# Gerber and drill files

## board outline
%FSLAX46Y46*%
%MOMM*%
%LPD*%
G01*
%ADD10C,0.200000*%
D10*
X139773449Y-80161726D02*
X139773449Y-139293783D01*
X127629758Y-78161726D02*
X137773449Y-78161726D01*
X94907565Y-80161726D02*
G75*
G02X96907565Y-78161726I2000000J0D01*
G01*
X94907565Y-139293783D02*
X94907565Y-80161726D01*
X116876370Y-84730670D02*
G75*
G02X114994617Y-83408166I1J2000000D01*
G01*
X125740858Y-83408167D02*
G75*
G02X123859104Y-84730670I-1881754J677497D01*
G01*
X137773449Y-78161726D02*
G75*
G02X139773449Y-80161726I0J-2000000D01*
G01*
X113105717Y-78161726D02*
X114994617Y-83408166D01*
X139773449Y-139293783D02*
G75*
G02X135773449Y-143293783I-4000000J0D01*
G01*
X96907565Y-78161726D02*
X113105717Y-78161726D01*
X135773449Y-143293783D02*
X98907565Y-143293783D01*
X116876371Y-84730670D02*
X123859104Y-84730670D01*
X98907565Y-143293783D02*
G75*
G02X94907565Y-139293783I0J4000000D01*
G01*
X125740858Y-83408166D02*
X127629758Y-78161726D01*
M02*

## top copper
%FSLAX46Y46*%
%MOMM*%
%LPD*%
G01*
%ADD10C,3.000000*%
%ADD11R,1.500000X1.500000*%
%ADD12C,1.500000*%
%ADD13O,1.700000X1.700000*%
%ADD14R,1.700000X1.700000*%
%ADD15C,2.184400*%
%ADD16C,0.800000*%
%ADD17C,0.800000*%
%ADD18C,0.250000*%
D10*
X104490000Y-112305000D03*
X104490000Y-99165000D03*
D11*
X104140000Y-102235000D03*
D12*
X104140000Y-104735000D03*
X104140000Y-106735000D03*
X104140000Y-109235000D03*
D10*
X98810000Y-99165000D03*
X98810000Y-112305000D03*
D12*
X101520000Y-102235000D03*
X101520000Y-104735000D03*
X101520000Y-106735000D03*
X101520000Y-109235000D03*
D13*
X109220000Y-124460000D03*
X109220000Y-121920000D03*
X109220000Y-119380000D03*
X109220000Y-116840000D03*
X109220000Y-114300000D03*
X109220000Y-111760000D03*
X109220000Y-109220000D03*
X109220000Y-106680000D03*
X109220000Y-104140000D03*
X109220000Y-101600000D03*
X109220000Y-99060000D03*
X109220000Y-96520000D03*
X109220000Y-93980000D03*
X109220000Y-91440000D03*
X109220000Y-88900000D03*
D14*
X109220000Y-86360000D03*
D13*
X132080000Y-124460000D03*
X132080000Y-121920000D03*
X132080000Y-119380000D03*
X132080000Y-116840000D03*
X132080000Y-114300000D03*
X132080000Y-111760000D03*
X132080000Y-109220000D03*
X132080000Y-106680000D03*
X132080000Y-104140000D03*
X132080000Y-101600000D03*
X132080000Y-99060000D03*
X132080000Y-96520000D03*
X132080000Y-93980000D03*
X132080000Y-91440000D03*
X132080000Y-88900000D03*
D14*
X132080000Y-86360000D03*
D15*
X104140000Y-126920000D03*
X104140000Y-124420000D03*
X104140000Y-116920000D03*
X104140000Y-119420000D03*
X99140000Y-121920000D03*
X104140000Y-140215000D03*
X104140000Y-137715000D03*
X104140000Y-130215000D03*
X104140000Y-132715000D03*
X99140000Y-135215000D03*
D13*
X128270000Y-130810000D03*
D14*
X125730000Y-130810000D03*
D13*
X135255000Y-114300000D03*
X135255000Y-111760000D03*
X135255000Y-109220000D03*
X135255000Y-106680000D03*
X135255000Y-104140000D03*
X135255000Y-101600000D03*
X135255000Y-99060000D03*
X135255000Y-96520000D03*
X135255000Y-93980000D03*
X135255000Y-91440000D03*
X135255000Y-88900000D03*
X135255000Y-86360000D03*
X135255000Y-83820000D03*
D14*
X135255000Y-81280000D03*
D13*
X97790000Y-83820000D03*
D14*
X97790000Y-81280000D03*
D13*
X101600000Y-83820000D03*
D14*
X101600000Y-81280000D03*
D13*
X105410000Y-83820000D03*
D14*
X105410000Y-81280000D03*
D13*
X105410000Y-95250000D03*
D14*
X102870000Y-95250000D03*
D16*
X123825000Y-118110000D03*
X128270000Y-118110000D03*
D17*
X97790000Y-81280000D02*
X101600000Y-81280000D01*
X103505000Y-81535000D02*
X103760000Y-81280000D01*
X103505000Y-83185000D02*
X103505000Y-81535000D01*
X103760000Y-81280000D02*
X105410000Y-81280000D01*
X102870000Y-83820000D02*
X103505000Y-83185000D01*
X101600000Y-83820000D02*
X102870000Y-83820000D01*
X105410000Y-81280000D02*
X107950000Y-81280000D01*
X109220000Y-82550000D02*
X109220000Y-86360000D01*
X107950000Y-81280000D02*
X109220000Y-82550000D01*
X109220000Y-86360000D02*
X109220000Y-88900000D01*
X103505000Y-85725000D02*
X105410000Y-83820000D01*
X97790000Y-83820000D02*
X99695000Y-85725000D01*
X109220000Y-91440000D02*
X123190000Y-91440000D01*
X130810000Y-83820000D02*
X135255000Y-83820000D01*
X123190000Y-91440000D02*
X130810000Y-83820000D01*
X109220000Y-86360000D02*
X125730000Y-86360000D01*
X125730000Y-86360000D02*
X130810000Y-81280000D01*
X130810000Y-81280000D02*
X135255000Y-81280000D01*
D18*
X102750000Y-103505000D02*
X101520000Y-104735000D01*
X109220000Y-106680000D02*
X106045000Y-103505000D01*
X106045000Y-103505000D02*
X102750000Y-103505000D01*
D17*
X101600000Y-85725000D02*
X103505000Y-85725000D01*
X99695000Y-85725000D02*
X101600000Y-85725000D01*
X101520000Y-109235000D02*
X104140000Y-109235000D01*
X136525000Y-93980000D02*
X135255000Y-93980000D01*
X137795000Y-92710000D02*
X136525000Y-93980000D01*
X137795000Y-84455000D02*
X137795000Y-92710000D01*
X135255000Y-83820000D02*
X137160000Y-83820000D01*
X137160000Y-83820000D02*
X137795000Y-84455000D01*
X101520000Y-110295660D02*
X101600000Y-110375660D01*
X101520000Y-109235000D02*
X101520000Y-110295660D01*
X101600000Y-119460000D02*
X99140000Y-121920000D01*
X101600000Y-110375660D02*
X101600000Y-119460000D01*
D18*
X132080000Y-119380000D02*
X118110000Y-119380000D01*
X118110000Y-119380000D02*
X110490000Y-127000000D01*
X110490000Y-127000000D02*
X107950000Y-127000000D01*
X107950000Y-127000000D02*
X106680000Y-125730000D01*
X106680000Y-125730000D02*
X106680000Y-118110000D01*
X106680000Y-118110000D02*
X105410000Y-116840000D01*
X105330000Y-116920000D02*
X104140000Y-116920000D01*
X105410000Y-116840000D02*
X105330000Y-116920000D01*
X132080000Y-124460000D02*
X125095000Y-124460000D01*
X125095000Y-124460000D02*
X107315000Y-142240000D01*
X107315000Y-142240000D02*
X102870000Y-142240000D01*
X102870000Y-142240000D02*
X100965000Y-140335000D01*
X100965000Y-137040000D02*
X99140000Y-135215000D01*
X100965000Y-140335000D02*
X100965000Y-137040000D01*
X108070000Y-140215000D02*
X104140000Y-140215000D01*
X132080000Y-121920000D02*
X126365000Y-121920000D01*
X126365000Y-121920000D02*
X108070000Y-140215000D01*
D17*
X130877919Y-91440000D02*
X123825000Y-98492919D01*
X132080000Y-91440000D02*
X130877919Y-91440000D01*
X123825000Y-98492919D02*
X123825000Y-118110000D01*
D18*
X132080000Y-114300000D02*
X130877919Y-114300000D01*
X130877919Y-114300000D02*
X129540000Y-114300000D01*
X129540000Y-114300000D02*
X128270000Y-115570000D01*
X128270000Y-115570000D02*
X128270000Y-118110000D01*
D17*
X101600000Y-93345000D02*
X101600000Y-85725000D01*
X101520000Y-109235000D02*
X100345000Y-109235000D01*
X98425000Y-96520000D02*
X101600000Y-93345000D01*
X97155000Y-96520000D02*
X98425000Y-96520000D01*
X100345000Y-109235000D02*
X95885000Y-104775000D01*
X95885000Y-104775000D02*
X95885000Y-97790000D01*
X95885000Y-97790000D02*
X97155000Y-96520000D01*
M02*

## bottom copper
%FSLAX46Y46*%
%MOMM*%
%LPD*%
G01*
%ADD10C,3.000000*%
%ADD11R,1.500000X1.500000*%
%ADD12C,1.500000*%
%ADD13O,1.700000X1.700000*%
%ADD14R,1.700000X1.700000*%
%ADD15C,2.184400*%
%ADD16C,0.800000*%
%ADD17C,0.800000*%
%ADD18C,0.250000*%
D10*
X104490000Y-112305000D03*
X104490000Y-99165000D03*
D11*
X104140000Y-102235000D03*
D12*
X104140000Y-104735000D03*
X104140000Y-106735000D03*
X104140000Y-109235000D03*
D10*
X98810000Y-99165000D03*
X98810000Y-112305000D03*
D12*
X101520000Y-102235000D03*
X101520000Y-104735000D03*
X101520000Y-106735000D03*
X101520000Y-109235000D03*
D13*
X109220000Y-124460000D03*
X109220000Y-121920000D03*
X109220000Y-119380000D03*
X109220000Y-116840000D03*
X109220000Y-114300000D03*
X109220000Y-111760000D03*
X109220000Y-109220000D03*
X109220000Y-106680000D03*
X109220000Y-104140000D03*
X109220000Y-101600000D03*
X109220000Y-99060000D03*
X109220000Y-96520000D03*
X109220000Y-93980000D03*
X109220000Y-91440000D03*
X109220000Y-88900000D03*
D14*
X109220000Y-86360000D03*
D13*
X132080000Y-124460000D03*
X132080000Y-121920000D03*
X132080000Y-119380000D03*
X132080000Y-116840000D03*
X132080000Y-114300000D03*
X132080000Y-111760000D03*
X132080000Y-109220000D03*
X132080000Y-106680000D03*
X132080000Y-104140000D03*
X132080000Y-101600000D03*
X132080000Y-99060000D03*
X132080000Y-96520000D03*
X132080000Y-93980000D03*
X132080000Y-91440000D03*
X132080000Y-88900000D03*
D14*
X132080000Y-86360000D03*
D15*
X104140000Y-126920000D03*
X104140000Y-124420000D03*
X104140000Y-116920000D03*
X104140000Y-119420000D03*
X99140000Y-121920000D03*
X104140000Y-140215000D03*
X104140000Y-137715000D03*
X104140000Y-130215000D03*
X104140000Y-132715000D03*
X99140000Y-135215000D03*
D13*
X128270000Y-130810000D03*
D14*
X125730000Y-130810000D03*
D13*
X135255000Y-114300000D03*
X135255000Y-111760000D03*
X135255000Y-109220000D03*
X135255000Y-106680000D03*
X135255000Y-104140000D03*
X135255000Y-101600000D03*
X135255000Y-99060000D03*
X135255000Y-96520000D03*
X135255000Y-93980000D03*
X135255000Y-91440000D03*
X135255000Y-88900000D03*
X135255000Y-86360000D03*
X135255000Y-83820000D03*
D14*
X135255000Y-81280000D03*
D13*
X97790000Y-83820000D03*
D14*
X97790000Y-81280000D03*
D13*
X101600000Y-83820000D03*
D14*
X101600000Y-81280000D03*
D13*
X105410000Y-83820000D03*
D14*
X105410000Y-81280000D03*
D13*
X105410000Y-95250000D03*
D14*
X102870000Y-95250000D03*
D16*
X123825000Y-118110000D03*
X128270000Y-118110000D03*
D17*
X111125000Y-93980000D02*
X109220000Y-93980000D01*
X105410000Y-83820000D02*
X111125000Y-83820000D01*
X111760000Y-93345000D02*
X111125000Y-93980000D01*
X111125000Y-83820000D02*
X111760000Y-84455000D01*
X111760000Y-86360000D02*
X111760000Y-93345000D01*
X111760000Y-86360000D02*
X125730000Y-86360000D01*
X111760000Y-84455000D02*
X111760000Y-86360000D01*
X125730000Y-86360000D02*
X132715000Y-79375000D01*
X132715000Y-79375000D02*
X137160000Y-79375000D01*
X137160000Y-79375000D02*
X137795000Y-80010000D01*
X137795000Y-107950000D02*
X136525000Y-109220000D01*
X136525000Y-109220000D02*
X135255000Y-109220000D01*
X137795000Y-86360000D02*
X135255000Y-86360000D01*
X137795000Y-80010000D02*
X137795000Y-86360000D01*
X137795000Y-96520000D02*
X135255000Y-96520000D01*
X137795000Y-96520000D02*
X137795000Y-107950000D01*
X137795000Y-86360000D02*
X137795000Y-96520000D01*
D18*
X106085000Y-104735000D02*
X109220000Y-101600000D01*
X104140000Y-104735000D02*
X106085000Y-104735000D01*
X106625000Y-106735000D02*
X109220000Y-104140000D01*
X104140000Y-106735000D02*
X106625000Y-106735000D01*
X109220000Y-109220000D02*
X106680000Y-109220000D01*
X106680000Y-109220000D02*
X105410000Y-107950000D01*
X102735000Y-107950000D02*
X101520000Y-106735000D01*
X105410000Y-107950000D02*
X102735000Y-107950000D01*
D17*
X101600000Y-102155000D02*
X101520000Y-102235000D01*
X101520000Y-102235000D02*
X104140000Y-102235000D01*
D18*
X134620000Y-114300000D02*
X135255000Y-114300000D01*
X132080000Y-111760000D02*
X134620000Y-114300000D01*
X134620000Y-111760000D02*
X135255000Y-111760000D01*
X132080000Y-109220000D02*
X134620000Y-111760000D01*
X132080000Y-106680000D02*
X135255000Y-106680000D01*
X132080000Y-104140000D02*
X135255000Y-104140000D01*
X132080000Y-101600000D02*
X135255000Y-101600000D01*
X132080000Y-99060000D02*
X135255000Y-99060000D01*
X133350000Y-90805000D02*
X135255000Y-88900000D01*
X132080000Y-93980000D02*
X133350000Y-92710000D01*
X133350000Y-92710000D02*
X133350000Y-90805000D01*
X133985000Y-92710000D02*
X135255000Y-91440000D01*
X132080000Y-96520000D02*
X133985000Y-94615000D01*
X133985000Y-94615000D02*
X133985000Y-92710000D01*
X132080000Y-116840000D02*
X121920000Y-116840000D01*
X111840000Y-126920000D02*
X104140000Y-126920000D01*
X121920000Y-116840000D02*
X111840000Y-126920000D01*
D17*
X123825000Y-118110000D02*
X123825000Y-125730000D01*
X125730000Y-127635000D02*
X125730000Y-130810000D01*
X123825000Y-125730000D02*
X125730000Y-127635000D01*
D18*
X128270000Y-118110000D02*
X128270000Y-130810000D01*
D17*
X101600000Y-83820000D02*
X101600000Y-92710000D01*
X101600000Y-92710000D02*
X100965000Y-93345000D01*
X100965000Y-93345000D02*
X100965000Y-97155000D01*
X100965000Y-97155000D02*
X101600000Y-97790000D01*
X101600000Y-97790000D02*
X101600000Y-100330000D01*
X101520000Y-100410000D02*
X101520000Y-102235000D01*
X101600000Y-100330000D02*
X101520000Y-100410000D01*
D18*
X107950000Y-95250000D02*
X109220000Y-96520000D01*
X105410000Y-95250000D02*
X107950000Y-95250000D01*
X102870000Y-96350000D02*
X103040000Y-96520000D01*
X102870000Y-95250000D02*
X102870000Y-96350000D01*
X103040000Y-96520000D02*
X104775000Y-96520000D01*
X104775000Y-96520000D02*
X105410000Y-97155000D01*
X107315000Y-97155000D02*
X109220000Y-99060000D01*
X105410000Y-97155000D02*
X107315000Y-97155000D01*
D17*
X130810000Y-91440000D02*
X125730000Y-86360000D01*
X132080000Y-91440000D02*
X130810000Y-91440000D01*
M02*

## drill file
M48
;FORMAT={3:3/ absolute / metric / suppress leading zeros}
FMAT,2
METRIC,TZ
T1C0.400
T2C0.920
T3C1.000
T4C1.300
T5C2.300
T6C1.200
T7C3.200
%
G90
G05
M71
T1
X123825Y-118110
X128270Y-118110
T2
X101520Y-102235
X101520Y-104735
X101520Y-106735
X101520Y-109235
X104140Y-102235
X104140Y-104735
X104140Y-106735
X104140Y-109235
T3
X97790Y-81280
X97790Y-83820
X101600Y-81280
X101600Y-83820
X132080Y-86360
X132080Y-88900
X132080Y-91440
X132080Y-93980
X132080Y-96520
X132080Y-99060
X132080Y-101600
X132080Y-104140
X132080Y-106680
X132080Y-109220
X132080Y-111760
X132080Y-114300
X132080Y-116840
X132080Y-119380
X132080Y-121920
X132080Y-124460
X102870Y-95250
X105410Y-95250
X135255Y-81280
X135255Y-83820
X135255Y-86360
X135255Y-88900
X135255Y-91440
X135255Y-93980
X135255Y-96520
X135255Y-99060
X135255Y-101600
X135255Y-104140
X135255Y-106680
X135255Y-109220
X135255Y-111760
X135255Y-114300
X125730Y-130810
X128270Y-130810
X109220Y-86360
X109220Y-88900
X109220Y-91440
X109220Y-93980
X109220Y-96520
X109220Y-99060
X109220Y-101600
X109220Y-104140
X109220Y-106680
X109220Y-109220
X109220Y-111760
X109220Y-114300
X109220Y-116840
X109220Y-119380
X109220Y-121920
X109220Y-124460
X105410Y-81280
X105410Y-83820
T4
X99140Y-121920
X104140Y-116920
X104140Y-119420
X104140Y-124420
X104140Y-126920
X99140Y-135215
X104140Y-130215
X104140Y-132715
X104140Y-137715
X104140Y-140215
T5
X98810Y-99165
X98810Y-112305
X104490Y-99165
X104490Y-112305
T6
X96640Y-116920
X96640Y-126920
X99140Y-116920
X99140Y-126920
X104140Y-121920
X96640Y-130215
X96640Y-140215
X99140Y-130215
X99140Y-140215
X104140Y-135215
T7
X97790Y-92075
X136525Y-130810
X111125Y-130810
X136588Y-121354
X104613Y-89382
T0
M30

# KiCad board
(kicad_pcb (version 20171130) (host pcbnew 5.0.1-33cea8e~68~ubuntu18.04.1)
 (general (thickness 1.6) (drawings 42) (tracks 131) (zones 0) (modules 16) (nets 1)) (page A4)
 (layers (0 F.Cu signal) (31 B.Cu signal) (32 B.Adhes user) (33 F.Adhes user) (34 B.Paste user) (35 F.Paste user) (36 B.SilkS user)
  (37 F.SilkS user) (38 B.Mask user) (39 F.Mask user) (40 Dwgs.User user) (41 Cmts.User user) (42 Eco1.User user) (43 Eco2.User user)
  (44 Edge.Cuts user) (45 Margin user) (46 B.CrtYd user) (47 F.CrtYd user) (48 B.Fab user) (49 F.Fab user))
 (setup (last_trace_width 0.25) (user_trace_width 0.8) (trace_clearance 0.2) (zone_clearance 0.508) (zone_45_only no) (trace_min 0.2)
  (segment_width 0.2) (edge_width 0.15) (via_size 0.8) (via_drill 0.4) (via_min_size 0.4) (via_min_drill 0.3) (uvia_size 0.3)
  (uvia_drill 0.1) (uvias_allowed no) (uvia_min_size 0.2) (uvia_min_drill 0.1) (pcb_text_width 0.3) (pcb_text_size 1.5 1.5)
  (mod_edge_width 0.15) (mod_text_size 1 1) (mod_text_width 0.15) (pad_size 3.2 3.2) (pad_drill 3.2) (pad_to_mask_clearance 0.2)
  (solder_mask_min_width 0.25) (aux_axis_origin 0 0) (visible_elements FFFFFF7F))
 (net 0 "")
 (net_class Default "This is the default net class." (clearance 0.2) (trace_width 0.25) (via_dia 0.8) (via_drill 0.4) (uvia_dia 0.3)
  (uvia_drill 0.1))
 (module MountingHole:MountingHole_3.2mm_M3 (layer F.Cu) (at 97.79 92.075)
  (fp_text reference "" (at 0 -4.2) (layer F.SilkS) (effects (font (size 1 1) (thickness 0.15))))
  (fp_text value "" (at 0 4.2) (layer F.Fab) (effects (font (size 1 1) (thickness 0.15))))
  (pad 1 np_thru_hole circle (at 0 0) (size 3.2 3.2) (drill 3.2) (layers *.Cu *.Mask)))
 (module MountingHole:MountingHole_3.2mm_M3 (layer F.Cu) (at 136.525 130.81)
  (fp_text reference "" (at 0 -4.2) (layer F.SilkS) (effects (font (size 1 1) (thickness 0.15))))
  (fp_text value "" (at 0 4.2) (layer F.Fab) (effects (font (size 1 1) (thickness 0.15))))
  (pad 1 np_thru_hole circle (at 0 0) (size 3.2 3.2) (drill 3.2) (layers *.Cu *.Mask)))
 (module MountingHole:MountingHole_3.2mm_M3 (layer F.Cu) (at 111.125 130.81)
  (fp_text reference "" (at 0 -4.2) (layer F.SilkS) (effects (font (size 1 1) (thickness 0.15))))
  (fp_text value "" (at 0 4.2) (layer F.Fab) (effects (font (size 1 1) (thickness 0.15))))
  (pad 1 np_thru_hole circle (at 0 0) (size 3.2 3.2) (drill 3.2) (layers *.Cu *.Mask)))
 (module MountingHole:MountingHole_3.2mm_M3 (layer F.Cu) (at 136.587912 121.353509)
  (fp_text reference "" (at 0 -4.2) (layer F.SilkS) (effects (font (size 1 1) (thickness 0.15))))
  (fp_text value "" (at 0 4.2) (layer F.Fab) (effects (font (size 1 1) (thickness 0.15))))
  (pad 1 np_thru_hole circle (at 0 0) (size 3.2 3.2) (drill 3.2) (layers *.Cu *.Mask)))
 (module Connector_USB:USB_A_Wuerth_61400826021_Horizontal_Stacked (layer F.Cu) (at 104.14 102.235 270)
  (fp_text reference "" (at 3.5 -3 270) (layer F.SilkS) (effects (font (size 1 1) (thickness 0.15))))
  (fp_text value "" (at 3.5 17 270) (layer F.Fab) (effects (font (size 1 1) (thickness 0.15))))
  (pad 9 thru_hole circle (at 10.07 -0.35 270) (size 3 3) (drill 2.3) (layers *.Cu *.Mask))
  (pad 9 thru_hole circle (at -3.07 -0.35 270) (size 3 3) (drill 2.3) (layers *.Cu *.Mask))
  (pad 1 thru_hole rect (at 0 0 270) (size 1.5 1.5) (drill 0.92) (layers *.Cu *.Mask))
  (pad 2 thru_hole circle (at 2.5 0 270) (size 1.5 1.5) (drill 0.92) (layers *.Cu *.Mask))
  (pad 3 thru_hole circle (at 4.5 0 270) (size 1.5 1.5) (drill 0.92) (layers *.Cu *.Mask))
  (pad 4 thru_hole circle (at 7 0 270) (size 1.5 1.5) (drill 0.92) (layers *.Cu *.Mask))
  (pad 9 thru_hole circle (at -3.07 5.33 270) (size 3 3) (drill 2.3) (layers *.Cu *.Mask))
  (pad 9 thru_hole circle (at 10.07 5.33 270) (size 3 3) (drill 2.3) (layers *.Cu *.Mask))
  (pad 5 thru_hole circle (at 0 2.62 270) (size 1.5 1.5) (drill 0.92) (layers *.Cu *.Mask))
  (pad 6 thru_hole circle (at 2.5 2.62 270) (size 1.5 1.5) (drill 0.92) (layers *.Cu *.Mask))
  (pad 7 thru_hole circle (at 4.5 2.62 270) (size 1.5 1.5) (drill 0.92) (layers *.Cu *.Mask))
  (pad 8 thru_hole circle (at 7 2.62 270) (size 1.5 1.5) (drill 0.92) (layers *.Cu *.Mask)))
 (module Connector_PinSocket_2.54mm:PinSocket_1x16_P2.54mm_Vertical (layer F.Cu) (at 109.22 86.36)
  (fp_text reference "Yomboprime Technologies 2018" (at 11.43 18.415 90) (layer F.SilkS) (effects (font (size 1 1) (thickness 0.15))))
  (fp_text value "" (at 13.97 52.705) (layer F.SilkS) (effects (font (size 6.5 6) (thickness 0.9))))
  (pad 16 thru_hole oval (at 0 38.1) (size 1.7 1.7) (drill 1) (layers *.Cu *.Mask))
  (pad 15 thru_hole oval (at 0 35.56) (size 1.7 1.7) (drill 1) (layers *.Cu *.Mask))
  (pad 14 thru_hole oval (at 0 33.02) (size 1.7 1.7) (drill 1) (layers *.Cu *.Mask))
  (pad 13 thru_hole oval (at 0 30.48) (size 1.7 1.7) (drill 1) (layers *.Cu *.Mask))
  (pad 12 thru_hole oval (at 0 27.94) (size 1.7 1.7) (drill 1) (layers *.Cu *.Mask))
  (pad 11 thru_hole oval (at 0 25.4) (size 1.7 1.7) (drill 1) (layers *.Cu *.Mask))
  (pad 10 thru_hole oval (at 0 22.86) (size 1.7 1.7) (drill 1) (layers *.Cu *.Mask))
  (pad 9 thru_hole oval (at 0 20.32) (size 1.7 1.7) (drill 1) (layers *.Cu *.Mask))
  (pad 8 thru_hole oval (at 0 17.78) (size 1.7 1.7) (drill 1) (layers *.Cu *.Mask))
  (pad 7 thru_hole oval (at 0 15.24) (size 1.7 1.7) (drill 1) (layers *.Cu *.Mask))
  (pad 6 thru_hole oval (at 0 12.7) (size 1.7 1.7) (drill 1) (layers *.Cu *.Mask))
  (pad 5 thru_hole oval (at 0 10.16) (size 1.7 1.7) (drill 1) (layers *.Cu *.Mask))
  (pad 4 thru_hole oval (at 0 7.62) (size 1.7 1.7) (drill 1) (layers *.Cu *.Mask))
  (pad 3 thru_hole oval (at 0 5.08) (size 1.7 1.7) (drill 1) (layers *.Cu *.Mask))
  (pad 2 thru_hole oval (at 0 2.54) (size 1.7 1.7) (drill 1) (layers *.Cu *.Mask))
  (pad 1 thru_hole rect (at 0 0) (size 1.7 1.7) (drill 1) (layers *.Cu *.Mask)))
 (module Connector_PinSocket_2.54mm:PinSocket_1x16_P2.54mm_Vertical (layer F.Cu) (at 132.08 86.36)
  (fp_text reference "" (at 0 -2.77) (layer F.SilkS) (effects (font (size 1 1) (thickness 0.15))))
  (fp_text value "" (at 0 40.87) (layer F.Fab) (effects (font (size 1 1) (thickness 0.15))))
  (pad 16 thru_hole oval (at 0 38.1) (size 1.7 1.7) (drill 1) (layers *.Cu *.Mask))
  (pad 15 thru_hole oval (at 0 35.56) (size 1.7 1.7) (drill 1) (layers *.Cu *.Mask))
  (pad 14 thru_hole oval (at 0 33.02) (size 1.7 1.7) (drill 1) (layers *.Cu *.Mask))
  (pad 13 thru_hole oval (at 0 30.48) (size 1.7 1.7) (drill 1) (layers *.Cu *.Mask))
  (pad 12 thru_hole oval (at 0 27.94) (size 1.7 1.7) (drill 1) (layers *.Cu *.Mask))
  (pad 11 thru_hole oval (at 0 25.4) (size 1.7 1.7) (drill 1) (layers *.Cu *.Mask))
  (pad 10 thru_hole oval (at 0 22.86) (size 1.7 1.7) (drill 1) (layers *.Cu *.Mask))
  (pad 9 thru_hole oval (at 0 20.32) (size 1.7 1.7) (drill 1) (layers *.Cu *.Mask))
  (pad 8 thru_hole oval (at 0 17.78) (size 1.7 1.7) (drill 1) (layers *.Cu *.Mask))
  (pad 7 thru_hole oval (at 0 15.24) (size 1.7 1.7) (drill 1) (layers *.Cu *.Mask))
  (pad 6 thru_hole oval (at 0 12.7) (size 1.7 1.7) (drill 1) (layers *.Cu *.Mask))
  (pad 5 thru_hole oval (at 0 10.16) (size 1.7 1.7) (drill 1) (layers *.Cu *.Mask))
  (pad 4 thru_hole oval (at 0 7.62) (size 1.7 1.7) (drill 1) (layers *.Cu *.Mask))
  (pad 3 thru_hole oval (at 0 5.08) (size 1.7 1.7) (drill 1) (layers *.Cu *.Mask))
  (pad 2 thru_hole oval (at 0 2.54) (size 1.7 1.7) (drill 1) (layers *.Cu *.Mask))
  (pad 1 thru_hole rect (at 0 0) (size 1.7 1.7) (drill 1) (layers *.Cu *.Mask)))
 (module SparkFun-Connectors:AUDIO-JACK (layer F.Cu) (at 99.14 121.92)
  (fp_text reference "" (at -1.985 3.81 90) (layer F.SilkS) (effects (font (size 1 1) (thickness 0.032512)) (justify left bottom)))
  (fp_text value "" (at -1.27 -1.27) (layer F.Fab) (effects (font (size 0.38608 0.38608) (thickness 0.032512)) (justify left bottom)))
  (pad "" np_thru_hole circle (at 5 0) (size 1.2 1.2) (drill 1.2) (layers *.Cu))
  (pad "" np_thru_hole circle (at 0 5) (size 1.2 1.2) (drill 1.2) (layers *.Cu))
  (pad "" np_thru_hole circle (at -2.5 5) (size 1.2 1.2) (drill 1.2) (layers *.Cu))
  (pad "" np_thru_hole circle (at -2.5 -5) (size 1.2 1.2) (drill 1.2) (layers *.Cu))
  (pad "" np_thru_hole circle (at 0 -5) (size 1.2 1.2) (drill 1.2) (layers *.Cu))
  (pad TIP thru_hole circle (at 5 5) (size 2.1844 2.1844) (drill 1.3) (layers *.Cu *.Mask) (solder_mask_margin 0.1016))
  (pad TSH thru_hole circle (at 5 2.5) (size 2.1844 2.1844) (drill 1.3) (layers *.Cu *.Mask) (solder_mask_margin 0.1016))
  (pad RING thru_hole circle (at 5 -5) (size 2.1844 2.1844) (drill 1.3) (layers *.Cu *.Mask) (solder_mask_margin 0.1016))
  (pad RSH thru_hole circle (at 5 -2.5) (size 2.1844 2.1844) (drill 1.3) (layers *.Cu *.Mask) (solder_mask_margin 0.1016))
  (pad SLEEVE thru_hole circle (at 0 0) (size 2.1844 2.1844) (drill 1.3) (layers *.Cu *.Mask) (solder_mask_margin 0.1016)))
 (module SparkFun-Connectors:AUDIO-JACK (layer F.Cu) (at 99.14 135.215)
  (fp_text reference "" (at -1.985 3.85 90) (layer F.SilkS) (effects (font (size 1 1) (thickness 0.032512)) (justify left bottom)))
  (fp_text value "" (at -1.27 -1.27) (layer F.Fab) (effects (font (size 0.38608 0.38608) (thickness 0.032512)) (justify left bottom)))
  (pad "" np_thru_hole circle (at 5 0) (size 1.2 1.2) (drill 1.2) (layers *.Cu))
  (pad "" np_thru_hole circle (at 0 5) (size 1.2 1.2) (drill 1.2) (layers *.Cu))
  (pad "" np_thru_hole circle (at -2.5 5) (size 1.2 1.2) (drill 1.2) (layers *.Cu))
  (pad "" np_thru_hole circle (at -2.5 -5) (size 1.2 1.2) (drill 1.2) (layers *.Cu))
  (pad "" np_thru_hole circle (at 0 -5) (size 1.2 1.2) (drill 1.2) (layers *.Cu))
  (pad TIP thru_hole circle (at 5 5) (size 2.1844 2.1844) (drill 1.3) (layers *.Cu *.Mask) (solder_mask_margin 0.1016))
  (pad TSH thru_hole circle (at 5 2.5) (size 2.1844 2.1844) (drill 1.3) (layers *.Cu *.Mask) (solder_mask_margin 0.1016))
  (pad RING thru_hole circle (at 5 -5) (size 2.1844 2.1844) (drill 1.3) (layers *.Cu *.Mask) (solder_mask_margin 0.1016))
  (pad RSH thru_hole circle (at 5 -2.5) (size 2.1844 2.1844) (drill 1.3) (layers *.Cu *.Mask) (solder_mask_margin 0.1016))
  (pad SLEEVE thru_hole circle (at 0 0) (size 2.1844 2.1844) (drill 1.3) (layers *.Cu *.Mask) (solder_mask_margin 0.1016)))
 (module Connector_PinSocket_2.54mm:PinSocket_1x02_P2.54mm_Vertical (layer F.Cu) (at 125.73 130.81 90)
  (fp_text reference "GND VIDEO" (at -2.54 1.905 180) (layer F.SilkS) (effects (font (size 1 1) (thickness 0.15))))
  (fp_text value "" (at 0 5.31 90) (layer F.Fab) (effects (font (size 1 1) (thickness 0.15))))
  (pad 2 thru_hole oval (at 0 2.54 90) (size 1.7 1.7) (drill 1) (layers *.Cu *.Mask))
  (pad 1 thru_hole rect (at 0 0 90) (size 1.7 1.7) (drill 1) (layers *.Cu *.Mask)))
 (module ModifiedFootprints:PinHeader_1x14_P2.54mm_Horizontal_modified (layer F.Cu) (at 135.255 81.28)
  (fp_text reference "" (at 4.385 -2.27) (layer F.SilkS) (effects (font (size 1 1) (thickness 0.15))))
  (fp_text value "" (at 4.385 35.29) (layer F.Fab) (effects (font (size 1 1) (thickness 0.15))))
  (pad 14 thru_hole oval (at 0 33.02) (size 1.7 1.7) (drill 1) (layers *.Cu *.Mask))
  (pad 13 thru_hole oval (at 0 30.48) (size 1.7 1.7) (drill 1) (layers *.Cu *.Mask))
  (pad 12 thru_hole oval (at 0 27.94) (size 1.7 1.7) (drill 1) (layers *.Cu *.Mask))
  (pad 11 thru_hole oval (at 0 25.4) (size 1.7 1.7) (drill 1) (layers *.Cu *.Mask))
  (pad 10 thru_hole oval (at 0 22.86) (size 1.7 1.7) (drill 1) (layers *.Cu *.Mask))
  (pad 9 thru_hole oval (at 0 20.32) (size 1.7 1.7) (drill 1) (layers *.Cu *.Mask))
  (pad 8 thru_hole oval (at 0 17.78) (size 1.7 1.7) (drill 1) (layers *.Cu *.Mask))
  (pad 7 thru_hole oval (at 0 15.24) (size 1.7 1.7) (drill 1) (layers *.Cu *.Mask))
  (pad 6 thru_hole oval (at 0 12.7) (size 1.7 1.7) (drill 1) (layers *.Cu *.Mask))
  (pad 5 thru_hole oval (at 0 10.16) (size 1.7 1.7) (drill 1) (layers *.Cu *.Mask))
  (pad 4 thru_hole oval (at 0 7.62) (size 1.7 1.7) (drill 1) (layers *.Cu *.Mask))
  (pad 3 thru_hole oval (at 0 5.08) (size 1.7 1.7) (drill 1) (layers *.Cu *.Mask))
  (pad 2 thru_hole oval (at 0 2.54) (size 1.7 1.7) (drill 1) (layers *.Cu *.Mask))
  (pad 1 thru_hole rect (at 0 0) (size 1.7 1.7) (drill 1) (layers *.Cu *.Mask)))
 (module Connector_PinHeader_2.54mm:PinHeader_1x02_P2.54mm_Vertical (layer F.Cu) (at 97.79 81.28)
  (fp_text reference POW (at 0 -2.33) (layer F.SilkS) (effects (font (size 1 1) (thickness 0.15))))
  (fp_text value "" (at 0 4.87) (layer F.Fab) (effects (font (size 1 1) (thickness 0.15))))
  (pad 2 thru_hole oval (at 0 2.54) (size 1.7 1.7) (drill 1) (layers *.Cu *.Mask))
  (pad 1 thru_hole rect (at 0 0) (size 1.7 1.7) (drill 1) (layers *.Cu *.Mask)))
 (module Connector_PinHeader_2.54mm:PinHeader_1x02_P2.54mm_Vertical (layer F.Cu) (at 101.6 81.28)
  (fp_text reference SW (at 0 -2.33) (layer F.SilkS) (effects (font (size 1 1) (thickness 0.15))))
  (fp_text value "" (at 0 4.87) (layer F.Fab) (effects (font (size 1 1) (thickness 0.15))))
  (pad 2 thru_hole oval (at 0 2.54) (size 1.7 1.7) (drill 1) (layers *.Cu *.Mask))
  (pad 1 thru_hole rect (at 0 0) (size 1.7 1.7) (drill 1) (layers *.Cu *.Mask)))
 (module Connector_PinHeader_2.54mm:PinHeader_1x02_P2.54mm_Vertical (layer F.Cu) (at 105.41 81.28)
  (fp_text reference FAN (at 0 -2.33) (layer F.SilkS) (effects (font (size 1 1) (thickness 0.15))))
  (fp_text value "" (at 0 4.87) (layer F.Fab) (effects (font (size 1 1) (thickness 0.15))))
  (pad 2 thru_hole oval (at 0 2.54) (size 1.7 1.7) (drill 1) (layers *.Cu *.Mask))
  (pad 1 thru_hole rect (at 0 0) (size 1.7 1.7) (drill 1) (layers *.Cu *.Mask)))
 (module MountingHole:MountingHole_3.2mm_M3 (layer F.Cu) (at 104.612601 89.382307)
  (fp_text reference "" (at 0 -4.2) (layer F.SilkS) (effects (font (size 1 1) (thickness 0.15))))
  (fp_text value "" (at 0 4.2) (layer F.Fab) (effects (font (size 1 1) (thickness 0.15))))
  (pad 1 np_thru_hole circle (at 0 0) (size 3.2 3.2) (drill 3.2) (layers *.Cu *.Mask)))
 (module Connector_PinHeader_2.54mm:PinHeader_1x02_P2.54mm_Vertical (layer F.Cu) (at 102.87 95.25 90)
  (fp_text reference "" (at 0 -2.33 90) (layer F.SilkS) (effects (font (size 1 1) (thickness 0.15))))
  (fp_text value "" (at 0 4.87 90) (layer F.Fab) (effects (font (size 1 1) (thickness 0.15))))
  (pad 2 thru_hole oval (at 0 2.54 90) (size 1.7 1.7) (drill 1) (layers *.Cu *.Mask))
  (pad 1 thru_hole rect (at 0 0 90) (size 1.7 1.7) (drill 1) (layers *.Cu *.Mask)))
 (gr_line (start 139.773449 80.161726) (end 139.773449 139.293783) (layer Edge.Cuts) (width 0.2))
 (gr_line (start 127.629758 78.161726) (end 137.773449 78.161726) (layer Edge.Cuts) (width 0.2))
 (gr_arc (start 96.907565 80.161726) (end 96.907565 78.161726) (angle -90) (layer Edge.Cuts) (width 0.2))
 (gr_line (start 94.907565 139.293783) (end 94.907565 80.161726) (layer Edge.Cuts) (width 0.2))
 (gr_arc (start 116.876371 82.73067) (end 114.994617 83.408166) (angle -70.19936805) (layer Edge.Cuts) (width 0.2))
 (gr_arc (start 123.859104 82.73067) (end 123.859104 84.73067) (angle -70.19936805) (layer Edge.Cuts) (width 0.2))
 (gr_arc (start 137.773449 80.161726) (end 139.773449 80.161726) (angle -90) (layer Edge.Cuts) (width 0.2))
 (gr_line (start 113.105717 78.161726) (end 114.994617 83.408166) (layer Edge.Cuts) (width 0.2))
 (gr_arc (start 135.773449 139.293783) (end 135.773449 143.293783) (angle -90) (layer Edge.Cuts) (width 0.2))
 (gr_line (start 96.907565 78.161726) (end 113.105717 78.161726) (layer Edge.Cuts) (width 0.2))
 (gr_line (start 135.773449 143.293783) (end 98.907565 143.293783) (layer Edge.Cuts) (width 0.2))
 (gr_line (start 116.876371 84.73067) (end 123.859104 84.73067) (layer Edge.Cuts) (width 0.2))
 (gr_arc (start 98.907565 139.293783) (end 94.907565 139.293783) (angle -90) (layer Edge.Cuts) (width 0.2))
 (gr_line (start 125.740858 83.408166) (end 127.629758 78.161726) (layer Edge.Cuts) (width 0.2))
 (segment (start 97.79 81.28) (end 101.6 81.28) (width 0.8) (layer F.Cu) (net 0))
 (segment (start 103.505 81.535) (end 103.76 81.28) (width 0.8) (layer F.Cu) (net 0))
 (segment (start 103.505 83.185) (end 103.505 81.535) (width 0.8) (layer F.Cu) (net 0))
 (segment (start 103.76 81.28) (end 105.41 81.28) (width 0.8) (layer F.Cu) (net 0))
 (segment (start 102.87 83.82) (end 103.505 83.185) (width 0.8) (layer F.Cu) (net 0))
 (segment (start 101.6 83.82) (end 102.87 83.82) (width 0.8) (layer F.Cu) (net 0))
 (segment (start 105.41 81.28) (end 107.95 81.28) (width 0.8) (layer F.Cu) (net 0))
 (segment (start 109.22 82.55) (end 109.22 86.36) (width 0.8) (layer F.Cu) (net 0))
 (segment (start 107.95 81.28) (end 109.22 82.55) (width 0.8) (layer F.Cu) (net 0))
 (segment (start 109.22 86.36) (end 109.22 88.9) (width 0.8) (layer F.Cu) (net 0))
 (segment (start 103.505 85.725) (end 105.41 83.82) (width 0.8) (layer F.Cu) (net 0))
 (segment (start 97.79 83.82) (end 99.695 85.725) (width 0.8) (layer F.Cu) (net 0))
 (segment (start 111.125 93.98) (end 109.22 93.98) (width 0.8) (layer B.Cu) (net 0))
 (segment (start 105.41 83.82) (end 111.125 83.82) (width 0.8) (layer B.Cu) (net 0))
 (segment (start 111.76 93.345) (end 111.125 93.98) (width 0.8) (layer B.Cu) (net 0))
 (segment (start 111.125 83.82) (end 111.76 84.455) (width 0.8) (layer B.Cu) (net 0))
 (segment (start 109.22 91.44) (end 123.19 91.44) (width 0.8) (layer F.Cu) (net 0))
 (segment (start 130.81 83.82) (end 135.255 83.82) (width 0.8) (layer F.Cu) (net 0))
 (segment (start 123.19 91.44) (end 130.81 83.82) (width 0.8) (layer F.Cu) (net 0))
 (segment (start 109.22 86.36) (end 125.73 86.36) (width 0.8) (layer F.Cu) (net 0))
 (segment (start 125.73 86.36) (end 130.81 81.28) (width 0.8) (layer F.Cu) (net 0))
 (segment (start 130.81 81.28) (end 135.255 81.28) (width 0.8) (layer F.Cu) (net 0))
 (segment (start 111.76 86.36) (end 111.76 93.345) (width 0.8) (layer B.Cu) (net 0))
 (segment (start 111.76 86.36) (end 125.73 86.36) (width 0.8) (layer B.Cu) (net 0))
 (segment (start 111.76 84.455) (end 111.76 86.36) (width 0.8) (layer B.Cu) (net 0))
 (segment (start 125.73 86.36) (end 132.715 79.375) (width 0.8) (layer B.Cu) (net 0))
 (segment (start 132.715 79.375) (end 137.16 79.375) (width 0.8) (layer B.Cu) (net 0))
 (segment (start 137.16 79.375) (end 137.795 80.01) (width 0.8) (layer B.Cu) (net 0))
 (segment (start 137.795 107.95) (end 136.525 109.22) (width 0.8) (layer B.Cu) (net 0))
 (segment (start 136.525 109.22) (end 135.255 109.22) (width 0.8) (layer B.Cu) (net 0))
 (segment (start 137.795 86.36) (end 135.255 86.36) (width 0.8) (layer B.Cu) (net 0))
 (segment (start 137.795 80.01) (end 137.795 86.36) (width 0.8) (layer B.Cu) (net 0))
 (segment (start 137.795 96.52) (end 135.255 96.52) (width 0.8) (layer B.Cu) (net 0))
 (segment (start 137.795 96.52) (end 137.795 107.95) (width 0.8) (layer B.Cu) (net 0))
 (segment (start 137.795 86.36) (end 137.795 96.52) (width 0.8) (layer B.Cu) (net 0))
 (segment (start 106.085 104.735) (end 109.22 101.6) (width 0.25) (layer B.Cu) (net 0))
 (segment (start 104.14 104.735) (end 106.085 104.735) (width 0.25) (layer B.Cu) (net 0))
 (segment (start 106.625 106.735) (end 109.22 104.14) (width 0.25) (layer B.Cu) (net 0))
 (segment (start 104.14 106.735) (end 106.625 106.735) (width 0.25) (layer B.Cu) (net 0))
 (segment (start 109.22 109.22) (end 106.68 109.22) (width 0.25) (layer B.Cu) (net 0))
 (segment (start 106.68 109.22) (end 105.41 107.95) (width 0.25) (layer B.Cu) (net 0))
 (segment (start 102.735 107.95) (end 101.52 106.735) (width 0.25) (layer B.Cu) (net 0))
 (segment (start 105.41 107.95) (end 102.735 107.95) (width 0.25) (layer B.Cu) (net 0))
 (segment (start 102.75 103.505) (end 101.52 104.735) (width 0.25) (layer F.Cu) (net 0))
 (segment (start 109.22 106.68) (end 106.045 103.505) (width 0.25) (layer F.Cu) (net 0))
 (segment (start 106.045 103.505) (end 102.75 103.505) (width 0.25) (layer F.Cu) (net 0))
 (segment (start 101.6 85.725) (end 103.505 85.725) (width 0.8) (layer F.Cu) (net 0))
 (segment (start 99.695 85.725) (end 101.6 85.725) (width 0.8) (layer F.Cu) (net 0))
 (segment (start 101.52 109.235) (end 104.14 109.235) (width 0.8) (layer F.Cu) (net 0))
 (segment (start 101.6 102.155) (end 101.52 102.235) (width 0.8) (layer B.Cu) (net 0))
 (segment (start 101.52 102.235) (end 104.14 102.235) (width 0.8) (layer B.Cu) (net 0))
 (segment (start 134.62 114.3) (end 135.255 114.3) (width 0.25) (layer B.Cu) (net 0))
 (segment (start 132.08 111.76) (end 134.62 114.3) (width 0.25) (layer B.Cu) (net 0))
 (segment (start 134.62 111.76) (end 135.255 111.76) (width 0.25) (layer B.Cu) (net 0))
 (segment (start 132.08 109.22) (end 134.62 111.76) (width 0.25) (layer B.Cu) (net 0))
 (segment (start 132.08 106.68) (end 135.255 106.68) (width 0.25) (layer B.Cu) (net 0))
 (segment (start 132.08 104.14) (end 135.255 104.14) (width 0.25) (layer B.Cu) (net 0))
 (segment (start 132.08 101.6) (end 135.255 101.6) (width 0.25) (layer B.Cu) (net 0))
 (segment (start 132.08 99.06) (end 135.255 99.06) (width 0.25) (layer B.Cu) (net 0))
 (segment (start 133.35 90.805) (end 135.255 88.9) (width 0.25) (layer B.Cu) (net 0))
 (segment (start 132.08 93.98) (end 133.35 92.71) (width 0.25) (layer B.Cu) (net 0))
 (segment (start 133.35 92.71) (end 133.35 90.805) (width 0.25) (layer B.Cu) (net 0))
 (segment (start 133.985 92.71) (end 135.255 91.44) (width 0.25) (layer B.Cu) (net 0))
 (segment (start 132.08 96.52) (end 133.985 94.615) (width 0.25) (layer B.Cu) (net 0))
 (segment (start 133.985 94.615) (end 133.985 92.71) (width 0.25) (layer B.Cu) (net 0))
 (segment (start 136.525 93.98) (end 135.255 93.98) (width 0.8) (layer F.Cu) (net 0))
 (segment (start 137.795 92.71) (end 136.525 93.98) (width 0.8) (layer F.Cu) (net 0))
 (segment (start 137.795 84.455) (end 137.795 92.71) (width 0.8) (layer F.Cu) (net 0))
 (segment (start 135.255 83.82) (end 137.16 83.82) (width 0.8) (layer F.Cu) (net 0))
 (segment (start 137.16 83.82) (end 137.795 84.455) (width 0.8) (layer F.Cu) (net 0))
 (segment (start 101.52 110.29566) (end 101.6 110.37566) (width 0.8) (layer F.Cu) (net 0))
 (segment (start 101.52 109.235) (end 101.52 110.29566) (width 0.8) (layer F.Cu) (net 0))
 (segment (start 101.6 119.46) (end 99.14 121.92) (width 0.8) (layer F.Cu) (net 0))
 (segment (start 101.6 110.37566) (end 101.6 119.46) (width 0.8) (layer F.Cu) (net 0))
 (segment (start 132.08 119.38) (end 118.11 119.38) (width 0.25) (layer F.Cu) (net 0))
 (segment (start 118.11 119.38) (end 110.49 127) (width 0.25) (layer F.Cu) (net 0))
 (segment (start 110.49 127) (end 107.95 127) (width 0.25) (layer F.Cu) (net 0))
 (segment (start 107.95 127) (end 106.68 125.73) (width 0.25) (layer F.Cu) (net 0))
 (segment (start 106.68 125.73) (end 106.68 118.11) (width 0.25) (layer F.Cu) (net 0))
 (segment (start 106.68 118.11) (end 105.41 116.84) (width 0.25) (layer F.Cu) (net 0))
 (segment (start 105.33 116.92) (end 104.14 116.92) (width 0.25) (layer F.Cu) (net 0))
 (segment (start 105.41 116.84) (end 105.33 116.92) (width 0.25) (layer F.Cu) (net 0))
 (segment (start 132.08 116.84) (end 121.92 116.84) (width 0.25) (layer B.Cu) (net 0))
 (segment (start 111.84 126.92) (end 104.14 126.92) (width 0.25) (layer B.Cu) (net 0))
 (segment (start 121.92 116.84) (end 111.84 126.92) (width 0.25) (layer B.Cu) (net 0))
 (segment (start 132.08 124.46) (end 125.095 124.46) (width 0.25) (layer F.Cu) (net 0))
 (segment (start 125.095 124.46) (end 107.315 142.24) (width 0.25) (layer F.Cu) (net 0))
 (segment (start 107.315 142.24) (end 102.87 142.24) (width 0.25) (layer F.Cu) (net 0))
 (segment (start 102.87 142.24) (end 100.965 140.335) (width 0.25) (layer F.Cu) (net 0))
 (segment (start 100.965 137.04) (end 99.14 135.215) (width 0.25) (layer F.Cu) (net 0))
 (segment (start 100.965 140.335) (end 100.965 137.04) (width 0.25) (layer F.Cu) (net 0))
 (segment (start 108.07 140.215) (end 104.14 140.215) (width 0.25) (layer F.Cu) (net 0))
 (segment (start 132.08 121.92) (end 126.365 121.92) (width 0.25) (layer F.Cu) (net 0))
 (segment (start 126.365 121.92) (end 108.07 140.215) (width 0.25) (layer F.Cu) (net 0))
 (segment (start 130.877919 91.44) (end 123.825 98.492919) (width 0.8) (layer F.Cu) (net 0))
 (segment (start 132.08 91.44) (end 130.877919 91.44) (width 0.8) (layer F.Cu) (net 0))
 (via (at 123.825 118.11) (size 0.8) (drill 0.4) (layers F.Cu B.Cu) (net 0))
 (segment (start 123.825 98.492919) (end 123.825 118.11) (width 0.8) (layer F.Cu) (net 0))
 (segment (start 123.825 118.11) (end 123.825 125.73) (width 0.8) (layer B.Cu) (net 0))
 (segment (start 125.73 127.635) (end 125.73 130.81) (width 0.8) (layer B.Cu) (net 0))
 (segment (start 123.825 125.73) (end 125.73 127.635) (width 0.8) (layer B.Cu) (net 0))
 (segment (start 132.08 114.3) (end 130.877919 114.3) (width 0.25) (layer F.Cu) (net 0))
 (segment (start 130.877919 114.3) (end 129.54 114.3) (width 0.25) (layer F.Cu) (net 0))
 (via (at 128.27 118.11) (size 0.8) (drill 0.4) (layers F.Cu B.Cu) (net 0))
 (segment (start 129.54 114.3) (end 128.27 115.57) (width 0.25) (layer F.Cu) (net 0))
 (segment (start 128.27 115.57) (end 128.27 118.11) (width 0.25) (layer F.Cu) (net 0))
 (segment (start 128.27 118.11) (end 128.27 130.81) (width 0.25) (layer B.Cu) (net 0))
 (segment (start 101.6 93.345) (end 101.6 85.725) (width 0.8) (layer F.Cu) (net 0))
 (segment (start 101.52 109.235) (end 100.345 109.235) (width 0.8) (layer F.Cu) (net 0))
 (segment (start 98.425 96.52) (end 101.6 93.345) (width 0.8) (layer F.Cu) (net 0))
 (segment (start 97.155 96.52) (end 98.425 96.52) (width 0.8) (layer F.Cu) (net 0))
 (segment (start 100.345 109.235) (end 95.885 104.775) (width 0.8) (layer F.Cu) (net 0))
 (segment (start 95.885 104.775) (end 95.885 97.79) (width 0.8) (layer F.Cu) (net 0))
 (segment (start 95.885 97.79) (end 97.155 96.52) (width 0.8) (layer F.Cu) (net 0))
 (segment (start 101.6 83.82) (end 101.6 92.71) (width 0.8) (layer B.Cu) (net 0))
 (segment (start 101.6 92.71) (end 100.965 93.345) (width 0.8) (layer B.Cu) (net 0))
 (segment (start 100.965 93.345) (end 100.965 97.155) (width 0.8) (layer B.Cu) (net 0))
 (segment (start 100.965 97.155) (end 101.6 97.79) (width 0.8) (layer B.Cu) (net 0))
 (segment (start 101.6 97.79) (end 101.6 100.33) (width 0.8) (layer B.Cu) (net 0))
 (segment (start 101.52 100.41) (end 101.52 102.235) (width 0.8) (layer B.Cu) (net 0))
 (segment (start 101.6 100.33) (end 101.52 100.41) (width 0.8) (layer B.Cu) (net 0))
 (segment (start 107.95 95.25) (end 109.22 96.52) (width 0.25) (layer B.Cu) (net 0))
 (segment (start 105.41 95.25) (end 107.95 95.25) (width 0.25) (layer B.Cu) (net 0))
 (segment (start 102.87 96.35) (end 103.04 96.52) (width 0.25) (layer B.Cu) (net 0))
 (segment (start 102.87 95.25) (end 102.87 96.35) (width 0.25) (layer B.Cu) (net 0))
 (segment (start 103.04 96.52) (end 104.775 96.52) (width 0.25) (layer B.Cu) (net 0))
 (segment (start 104.775 96.52) (end 105.41 97.155) (width 0.25) (layer B.Cu) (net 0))
 (segment (start 107.315 97.155) (end 109.22 99.06) (width 0.25) (layer B.Cu) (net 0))
 (segment (start 105.41 97.155) (end 107.315 97.155) (width 0.25) (layer B.Cu) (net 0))
 (segment (start 130.81 91.44) (end 125.73 86.36) (width 0.8) (layer B.Cu) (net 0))
 (segment (start 132.08 91.44) (end 130.81 91.44) (width 0.8) (layer B.Cu) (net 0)))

